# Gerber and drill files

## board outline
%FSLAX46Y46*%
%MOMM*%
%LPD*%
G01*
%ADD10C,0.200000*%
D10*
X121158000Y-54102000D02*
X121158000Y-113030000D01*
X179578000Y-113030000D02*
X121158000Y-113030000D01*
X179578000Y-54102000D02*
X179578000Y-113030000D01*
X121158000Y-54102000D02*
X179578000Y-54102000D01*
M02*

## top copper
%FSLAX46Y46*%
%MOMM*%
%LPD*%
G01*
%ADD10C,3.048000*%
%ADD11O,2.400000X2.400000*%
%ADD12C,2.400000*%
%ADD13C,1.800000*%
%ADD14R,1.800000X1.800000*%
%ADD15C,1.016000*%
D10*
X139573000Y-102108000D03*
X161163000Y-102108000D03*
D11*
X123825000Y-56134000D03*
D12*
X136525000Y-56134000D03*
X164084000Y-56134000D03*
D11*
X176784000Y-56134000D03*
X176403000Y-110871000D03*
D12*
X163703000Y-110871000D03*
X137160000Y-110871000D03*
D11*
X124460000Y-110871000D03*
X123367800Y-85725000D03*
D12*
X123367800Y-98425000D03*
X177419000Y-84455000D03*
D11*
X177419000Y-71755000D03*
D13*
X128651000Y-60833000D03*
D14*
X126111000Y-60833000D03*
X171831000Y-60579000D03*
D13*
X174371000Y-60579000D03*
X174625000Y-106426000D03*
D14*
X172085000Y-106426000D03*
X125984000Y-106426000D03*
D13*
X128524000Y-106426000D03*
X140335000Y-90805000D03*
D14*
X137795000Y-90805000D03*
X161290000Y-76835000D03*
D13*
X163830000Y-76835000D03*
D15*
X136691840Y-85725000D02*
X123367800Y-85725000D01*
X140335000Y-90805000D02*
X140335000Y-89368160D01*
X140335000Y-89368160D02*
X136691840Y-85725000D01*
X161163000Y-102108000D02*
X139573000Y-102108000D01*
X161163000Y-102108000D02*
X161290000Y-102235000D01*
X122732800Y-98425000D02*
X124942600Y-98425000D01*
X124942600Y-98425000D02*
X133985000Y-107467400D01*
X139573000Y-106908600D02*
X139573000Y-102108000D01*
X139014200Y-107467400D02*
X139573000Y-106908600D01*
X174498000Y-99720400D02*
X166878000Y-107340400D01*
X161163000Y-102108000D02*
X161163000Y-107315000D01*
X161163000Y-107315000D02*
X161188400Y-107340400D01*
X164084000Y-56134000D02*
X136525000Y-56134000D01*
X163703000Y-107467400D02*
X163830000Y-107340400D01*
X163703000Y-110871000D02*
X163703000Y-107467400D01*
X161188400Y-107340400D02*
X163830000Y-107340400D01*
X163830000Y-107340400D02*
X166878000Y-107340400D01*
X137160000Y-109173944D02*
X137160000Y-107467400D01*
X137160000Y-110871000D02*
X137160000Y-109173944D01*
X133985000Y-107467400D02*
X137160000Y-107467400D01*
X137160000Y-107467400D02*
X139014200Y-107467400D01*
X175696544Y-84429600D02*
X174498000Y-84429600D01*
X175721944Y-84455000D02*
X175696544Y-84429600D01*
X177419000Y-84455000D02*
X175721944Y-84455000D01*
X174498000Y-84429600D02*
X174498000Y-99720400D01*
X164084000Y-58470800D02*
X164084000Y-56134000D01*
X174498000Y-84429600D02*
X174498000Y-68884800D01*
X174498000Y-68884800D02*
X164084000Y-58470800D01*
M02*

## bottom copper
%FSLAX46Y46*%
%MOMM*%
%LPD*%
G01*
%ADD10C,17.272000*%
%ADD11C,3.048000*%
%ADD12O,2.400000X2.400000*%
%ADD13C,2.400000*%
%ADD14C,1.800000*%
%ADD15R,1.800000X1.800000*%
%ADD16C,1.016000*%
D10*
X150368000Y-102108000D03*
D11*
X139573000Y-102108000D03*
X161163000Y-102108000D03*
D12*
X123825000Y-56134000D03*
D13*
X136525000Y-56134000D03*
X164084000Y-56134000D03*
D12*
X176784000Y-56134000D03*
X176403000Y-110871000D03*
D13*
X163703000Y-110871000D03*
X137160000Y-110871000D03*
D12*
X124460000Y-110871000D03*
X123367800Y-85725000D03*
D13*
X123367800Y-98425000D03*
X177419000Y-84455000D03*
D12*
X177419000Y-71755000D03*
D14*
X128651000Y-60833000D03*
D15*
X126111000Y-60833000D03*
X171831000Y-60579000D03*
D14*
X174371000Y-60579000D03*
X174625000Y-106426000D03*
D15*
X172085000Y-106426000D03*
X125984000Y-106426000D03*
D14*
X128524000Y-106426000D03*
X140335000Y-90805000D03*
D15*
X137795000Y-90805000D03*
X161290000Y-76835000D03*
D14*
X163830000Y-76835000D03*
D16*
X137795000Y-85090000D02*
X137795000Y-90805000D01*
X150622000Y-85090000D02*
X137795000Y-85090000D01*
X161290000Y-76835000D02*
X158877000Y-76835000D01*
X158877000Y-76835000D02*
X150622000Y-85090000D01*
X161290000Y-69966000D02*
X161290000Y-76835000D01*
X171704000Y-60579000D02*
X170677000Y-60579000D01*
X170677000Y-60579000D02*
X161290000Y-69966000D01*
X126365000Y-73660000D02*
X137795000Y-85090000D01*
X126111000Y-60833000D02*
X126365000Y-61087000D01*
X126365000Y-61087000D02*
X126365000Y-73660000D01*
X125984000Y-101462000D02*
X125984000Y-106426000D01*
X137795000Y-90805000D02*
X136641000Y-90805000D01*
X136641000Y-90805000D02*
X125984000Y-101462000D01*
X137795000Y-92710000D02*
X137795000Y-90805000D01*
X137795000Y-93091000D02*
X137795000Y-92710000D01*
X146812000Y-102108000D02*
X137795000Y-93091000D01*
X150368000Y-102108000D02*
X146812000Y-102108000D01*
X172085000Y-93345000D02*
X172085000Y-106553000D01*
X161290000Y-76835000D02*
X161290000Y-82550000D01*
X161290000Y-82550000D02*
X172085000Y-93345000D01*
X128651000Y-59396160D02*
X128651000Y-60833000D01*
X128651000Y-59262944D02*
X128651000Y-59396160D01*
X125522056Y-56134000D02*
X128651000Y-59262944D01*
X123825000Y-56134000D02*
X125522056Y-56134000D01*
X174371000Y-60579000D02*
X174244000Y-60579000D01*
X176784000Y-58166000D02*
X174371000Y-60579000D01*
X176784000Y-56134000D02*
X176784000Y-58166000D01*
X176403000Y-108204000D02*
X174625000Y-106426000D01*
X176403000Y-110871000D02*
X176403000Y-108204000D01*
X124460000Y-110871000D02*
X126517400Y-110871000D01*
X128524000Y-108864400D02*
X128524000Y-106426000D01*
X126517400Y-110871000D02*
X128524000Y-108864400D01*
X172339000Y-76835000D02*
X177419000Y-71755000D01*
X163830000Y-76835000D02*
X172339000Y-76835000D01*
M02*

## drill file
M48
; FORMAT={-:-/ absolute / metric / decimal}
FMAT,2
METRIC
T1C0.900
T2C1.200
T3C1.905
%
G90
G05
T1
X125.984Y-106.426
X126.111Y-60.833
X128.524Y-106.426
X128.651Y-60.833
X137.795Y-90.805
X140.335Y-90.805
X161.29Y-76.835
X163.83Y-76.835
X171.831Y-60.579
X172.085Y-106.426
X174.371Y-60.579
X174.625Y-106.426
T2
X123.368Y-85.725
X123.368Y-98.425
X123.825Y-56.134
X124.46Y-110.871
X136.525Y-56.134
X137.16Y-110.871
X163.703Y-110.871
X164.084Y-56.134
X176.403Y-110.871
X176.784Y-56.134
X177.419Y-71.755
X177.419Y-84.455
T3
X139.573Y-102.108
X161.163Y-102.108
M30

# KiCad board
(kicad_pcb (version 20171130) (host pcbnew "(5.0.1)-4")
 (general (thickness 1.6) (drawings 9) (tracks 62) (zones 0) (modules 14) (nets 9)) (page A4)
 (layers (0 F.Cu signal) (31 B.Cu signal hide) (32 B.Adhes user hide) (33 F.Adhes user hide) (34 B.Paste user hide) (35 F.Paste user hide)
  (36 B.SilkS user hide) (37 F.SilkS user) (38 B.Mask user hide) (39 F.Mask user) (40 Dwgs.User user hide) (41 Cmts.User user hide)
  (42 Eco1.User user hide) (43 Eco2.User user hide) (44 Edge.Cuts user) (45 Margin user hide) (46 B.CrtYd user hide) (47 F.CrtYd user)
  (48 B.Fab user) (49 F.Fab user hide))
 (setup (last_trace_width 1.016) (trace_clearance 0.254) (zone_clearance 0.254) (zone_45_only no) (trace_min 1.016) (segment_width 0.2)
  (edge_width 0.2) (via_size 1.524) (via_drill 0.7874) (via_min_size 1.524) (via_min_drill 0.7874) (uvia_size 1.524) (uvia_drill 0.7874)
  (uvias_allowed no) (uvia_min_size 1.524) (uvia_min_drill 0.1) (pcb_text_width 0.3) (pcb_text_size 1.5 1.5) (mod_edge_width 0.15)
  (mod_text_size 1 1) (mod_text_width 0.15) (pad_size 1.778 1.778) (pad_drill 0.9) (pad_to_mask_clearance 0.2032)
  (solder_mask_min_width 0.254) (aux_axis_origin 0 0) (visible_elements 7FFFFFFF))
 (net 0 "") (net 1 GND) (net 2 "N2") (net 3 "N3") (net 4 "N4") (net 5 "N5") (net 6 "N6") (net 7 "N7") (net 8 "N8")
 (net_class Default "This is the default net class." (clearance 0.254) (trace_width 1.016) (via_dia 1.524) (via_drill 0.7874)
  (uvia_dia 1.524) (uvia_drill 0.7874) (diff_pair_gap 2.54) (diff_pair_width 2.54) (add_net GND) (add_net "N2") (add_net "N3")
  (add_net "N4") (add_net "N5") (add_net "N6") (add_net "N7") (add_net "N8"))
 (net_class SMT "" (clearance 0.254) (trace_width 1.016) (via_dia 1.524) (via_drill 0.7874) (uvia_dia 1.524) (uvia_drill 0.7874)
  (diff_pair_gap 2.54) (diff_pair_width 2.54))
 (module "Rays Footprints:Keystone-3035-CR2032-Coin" (layer B.Cu) (at 150.368 102.108 180)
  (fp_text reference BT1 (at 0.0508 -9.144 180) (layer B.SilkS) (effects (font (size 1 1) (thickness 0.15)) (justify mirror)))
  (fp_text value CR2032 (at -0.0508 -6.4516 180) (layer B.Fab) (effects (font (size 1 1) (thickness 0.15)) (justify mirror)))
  (pad 2 smd circle (at 0 0 180) (size 17.272 17.272) (layers B.Cu B.Paste B.Mask) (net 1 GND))
  (pad 1 thru_hole circle (at 10.795 0 180) (size 3.048 3.048) (drill 1.905) (layers *.Cu *.Mask) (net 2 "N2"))
  (pad 1 thru_hole circle (at -10.795 0 90) (size 3.048 3.048) (drill 1.905) (layers *.Cu *.Mask) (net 2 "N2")))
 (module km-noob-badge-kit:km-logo (layer F.Cu) (at 150.368 83.566)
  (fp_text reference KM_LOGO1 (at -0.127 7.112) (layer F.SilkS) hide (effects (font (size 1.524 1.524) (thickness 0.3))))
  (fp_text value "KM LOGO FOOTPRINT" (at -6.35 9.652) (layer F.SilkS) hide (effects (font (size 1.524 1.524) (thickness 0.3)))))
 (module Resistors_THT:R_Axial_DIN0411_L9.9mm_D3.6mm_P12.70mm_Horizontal (layer F.Cu) (at 136.525 56.134 180)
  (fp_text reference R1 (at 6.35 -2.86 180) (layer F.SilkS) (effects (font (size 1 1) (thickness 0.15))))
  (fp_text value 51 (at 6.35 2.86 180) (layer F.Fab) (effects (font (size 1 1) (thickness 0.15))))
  (pad 2 thru_hole oval (at 12.7 0 180) (size 2.4 2.4) (drill 1.2) (layers *.Cu *.Mask) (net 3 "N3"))
  (pad 1 thru_hole circle (at 0 0 180) (size 2.4 2.4) (drill 1.2) (layers *.Cu *.Mask) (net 2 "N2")))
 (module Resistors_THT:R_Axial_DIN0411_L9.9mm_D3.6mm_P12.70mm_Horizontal (layer F.Cu) (at 164.084 56.134)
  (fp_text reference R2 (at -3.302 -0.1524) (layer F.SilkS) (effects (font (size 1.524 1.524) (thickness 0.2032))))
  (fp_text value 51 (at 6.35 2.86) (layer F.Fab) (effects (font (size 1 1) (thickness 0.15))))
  (pad 1 thru_hole circle (at 0 0) (size 2.4 2.4) (drill 1.2) (layers *.Cu *.Mask) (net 2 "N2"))
  (pad 2 thru_hole oval (at 12.7 0) (size 2.4 2.4) (drill 1.2) (layers *.Cu *.Mask) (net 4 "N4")))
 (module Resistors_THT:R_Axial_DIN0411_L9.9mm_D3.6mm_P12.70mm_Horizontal (layer F.Cu) (at 163.703 110.871)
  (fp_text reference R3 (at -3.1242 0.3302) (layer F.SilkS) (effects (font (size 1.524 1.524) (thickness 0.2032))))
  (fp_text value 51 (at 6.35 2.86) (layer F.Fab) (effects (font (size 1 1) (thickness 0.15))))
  (pad 2 thru_hole oval (at 12.7 0) (size 2.4 2.4) (drill 1.2) (layers *.Cu *.Mask) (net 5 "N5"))
  (pad 1 thru_hole circle (at 0 0) (size 2.4 2.4) (drill 1.2) (layers *.Cu *.Mask) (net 2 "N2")))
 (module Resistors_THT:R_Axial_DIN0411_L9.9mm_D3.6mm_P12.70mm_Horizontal (layer F.Cu) (at 137.16 110.871 180)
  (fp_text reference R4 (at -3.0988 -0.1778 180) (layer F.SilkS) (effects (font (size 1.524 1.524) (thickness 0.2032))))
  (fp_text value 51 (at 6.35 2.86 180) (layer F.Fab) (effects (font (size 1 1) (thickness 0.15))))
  (pad 1 thru_hole circle (at 0 0 180) (size 2.4 2.4) (drill 1.2) (layers *.Cu *.Mask) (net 2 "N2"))
  (pad 2 thru_hole oval (at 12.7 0 180) (size 2.4 2.4) (drill 1.2) (layers *.Cu *.Mask) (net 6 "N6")))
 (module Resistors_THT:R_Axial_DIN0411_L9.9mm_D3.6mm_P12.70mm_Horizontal (layer F.Cu) (at 123.3678 98.425 90)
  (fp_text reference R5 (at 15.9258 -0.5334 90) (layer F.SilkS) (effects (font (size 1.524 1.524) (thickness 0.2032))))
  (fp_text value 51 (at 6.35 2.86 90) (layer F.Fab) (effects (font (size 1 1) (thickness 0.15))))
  (pad 2 thru_hole oval (at 12.7 0 90) (size 2.4 2.4) (drill 1.2) (layers *.Cu *.Mask) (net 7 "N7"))
  (pad 1 thru_hole circle (at 0 0 90) (size 2.4 2.4) (drill 1.2) (layers *.Cu *.Mask) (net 2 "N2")))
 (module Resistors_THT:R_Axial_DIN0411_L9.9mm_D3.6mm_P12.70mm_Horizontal (layer F.Cu) (at 177.419 84.455 90)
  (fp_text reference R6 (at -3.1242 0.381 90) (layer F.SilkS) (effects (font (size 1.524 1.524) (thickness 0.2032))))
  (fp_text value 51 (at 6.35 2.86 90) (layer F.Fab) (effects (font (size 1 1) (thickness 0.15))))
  (pad 1 thru_hole circle (at 0 0 90) (size 2.4 2.4) (drill 1.2) (layers *.Cu *.Mask) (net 2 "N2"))
  (pad 2 thru_hole oval (at 12.7 0 90) (size 2.4 2.4) (drill 1.2) (layers *.Cu *.Mask) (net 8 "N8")))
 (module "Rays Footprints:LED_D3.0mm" (layer F.Cu) (at 126.111 60.833)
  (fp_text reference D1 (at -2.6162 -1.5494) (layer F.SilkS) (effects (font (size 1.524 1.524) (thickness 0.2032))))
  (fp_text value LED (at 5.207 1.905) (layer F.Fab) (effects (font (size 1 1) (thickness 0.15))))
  (pad 2 thru_hole circle (at 2.54 0) (size 1.8 1.8) (drill 0.9) (layers *.Cu *.Mask) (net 3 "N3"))
  (pad 1 thru_hole rect (at 0 0) (size 1.8 1.8) (drill 0.9) (layers *.Cu *.Mask) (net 1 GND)))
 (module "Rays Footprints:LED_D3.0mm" (layer F.Cu) (at 171.831 60.579)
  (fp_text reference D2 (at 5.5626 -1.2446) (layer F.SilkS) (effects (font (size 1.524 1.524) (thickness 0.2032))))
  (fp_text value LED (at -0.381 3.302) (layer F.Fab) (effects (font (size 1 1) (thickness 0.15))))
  (pad 1 thru_hole rect (at 0 0) (size 1.8 1.8) (drill 0.9) (layers *.Cu *.Mask) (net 1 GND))
  (pad 2 thru_hole circle (at 2.54 0) (size 1.8 1.8) (drill 0.9) (layers *.Cu *.Mask) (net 4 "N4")))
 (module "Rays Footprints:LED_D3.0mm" (layer F.Cu) (at 172.085 106.426)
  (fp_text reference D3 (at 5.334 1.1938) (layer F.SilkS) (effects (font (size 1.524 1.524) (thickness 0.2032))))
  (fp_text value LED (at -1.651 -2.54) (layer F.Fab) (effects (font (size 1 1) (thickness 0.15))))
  (pad 2 thru_hole circle (at 2.54 0) (size 1.8 1.8) (drill 0.9) (layers *.Cu *.Mask) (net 5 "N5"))
  (pad 1 thru_hole rect (at 0 0) (size 1.8 1.8) (drill 0.9) (layers *.Cu *.Mask) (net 1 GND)))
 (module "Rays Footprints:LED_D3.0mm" (layer F.Cu) (at 125.984 106.426)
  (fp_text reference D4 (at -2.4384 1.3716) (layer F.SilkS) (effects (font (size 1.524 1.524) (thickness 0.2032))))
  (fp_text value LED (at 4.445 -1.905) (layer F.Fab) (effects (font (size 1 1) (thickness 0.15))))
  (pad 1 thru_hole rect (at 0 0) (size 1.8 1.8) (drill 0.9) (layers *.Cu *.Mask) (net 1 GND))
  (pad 2 thru_hole circle (at 2.54 0) (size 1.8 1.8) (drill 0.9) (layers *.Cu *.Mask) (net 6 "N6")))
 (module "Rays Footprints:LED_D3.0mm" (layer F.Cu) (at 137.795 90.805)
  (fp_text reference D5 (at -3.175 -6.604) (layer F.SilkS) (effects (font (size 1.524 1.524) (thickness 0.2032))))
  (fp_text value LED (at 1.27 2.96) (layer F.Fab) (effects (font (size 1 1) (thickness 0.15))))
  (pad 2 thru_hole circle (at 2.54 0) (size 1.8 1.8) (drill 0.9) (layers *.Cu *.Mask) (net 7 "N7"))
  (pad 1 thru_hole rect (at 0 0) (size 1.8 1.8) (drill 0.9) (layers *.Cu *.Mask) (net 1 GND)))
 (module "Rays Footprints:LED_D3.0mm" (layer F.Cu) (at 161.29 76.835)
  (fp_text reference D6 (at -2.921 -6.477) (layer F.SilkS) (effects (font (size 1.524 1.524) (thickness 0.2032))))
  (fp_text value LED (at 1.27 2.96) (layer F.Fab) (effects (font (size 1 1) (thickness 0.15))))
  (pad 1 thru_hole rect (at 0 0) (size 1.8 1.8) (drill 0.9) (layers *.Cu *.Mask) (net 1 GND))
  (pad 2 thru_hole circle (at 2.54 0) (size 1.8 1.8) (drill 0.9) (layers *.Cu *.Mask) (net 8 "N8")))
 (gr_line (start 121.158 54.102) (end 121.158 113.03) (layer Edge.Cuts) (width 0.2))
 (gr_line (start 179.578 113.03) (end 121.158 113.03) (layer Edge.Cuts) (width 0.2))
 (gr_line (start 179.578 54.102) (end 179.578 113.03) (layer Edge.Cuts) (width 0.2))
 (gr_line (start 121.158 54.102) (end 179.578 54.102) (layer Edge.Cuts) (width 0.2))
 (segment (start 137.795 85.09) (end 137.795 90.805) (width 1.016) (layer B.Cu) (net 1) (status 20))
 (segment (start 150.622 85.09) (end 137.795 85.09) (width 1.016) (layer B.Cu) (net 1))
 (segment (start 161.29 76.835) (end 158.877 76.835) (width 1.016) (layer B.Cu) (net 1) (status 10))
 (segment (start 158.877 76.835) (end 150.622 85.09) (width 1.016) (layer B.Cu) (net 1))
 (segment (start 161.29 69.966) (end 161.29 76.835) (width 1.016) (layer B.Cu) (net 1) (status 20))
 (segment (start 171.704 60.579) (end 170.677 60.579) (width 1.016) (layer B.Cu) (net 1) (status 10))
 (segment (start 170.677 60.579) (end 161.29 69.966) (width 1.016) (layer B.Cu) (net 1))
 (segment (start 126.365 73.66) (end 137.795 85.09) (width 1.016) (layer B.Cu) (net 1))
 (segment (start 126.111 60.833) (end 126.365 61.087) (width 1.016) (layer B.Cu) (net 1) (status 30))
 (segment (start 126.365 61.087) (end 126.365 73.66) (width 1.016) (layer B.Cu) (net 1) (status 10))
 (segment (start 125.984 101.462) (end 125.984 106.426) (width 1.016) (layer B.Cu) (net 1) (status 20))
 (segment (start 137.795 90.805) (end 136.641 90.805) (width 1.016) (layer B.Cu) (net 1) (status 10))
 (segment (start 136.641 90.805) (end 125.984 101.462) (width 1.016) (layer B.Cu) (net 1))
 (segment (start 137.795 92.71) (end 137.795 90.805) (width 1.016) (layer B.Cu) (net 1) (status 20))
 (segment (start 137.795 93.091) (end 137.795 92.71) (width 1.016) (layer B.Cu) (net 1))
 (segment (start 146.812 102.108) (end 137.795 93.091) (width 1.016) (layer B.Cu) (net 1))
 (segment (start 150.368 102.108) (end 146.812 102.108) (width 1.016) (layer B.Cu) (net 1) (status 10))
 (segment (start 172.085 93.345) (end 172.085 106.553) (width 1.016) (layer B.Cu) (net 1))
 (segment (start 161.29 76.835) (end 161.29 82.55) (width 1.016) (layer B.Cu) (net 1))
 (segment (start 161.29 82.55) (end 172.085 93.345) (width 1.016) (layer B.Cu) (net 1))
 (segment (start 128.651 59.39616) (end 128.651 60.833) (width 1.016) (layer B.Cu) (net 3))
 (segment (start 128.651 59.262944) (end 128.651 59.39616) (width 1.016) (layer B.Cu) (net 3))
 (segment (start 125.522056 56.134) (end 128.651 59.262944) (width 1.016) (layer B.Cu) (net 3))
 (segment (start 123.825 56.134) (end 125.522056 56.134) (width 1.016) (layer B.Cu) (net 3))
 (segment (start 174.371 60.579) (end 174.244 60.579) (width 1.016) (layer B.Cu) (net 4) (status 30))
 (segment (start 176.784 58.166) (end 174.371 60.579) (width 1.016) (layer B.Cu) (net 4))
 (segment (start 176.784 56.134) (end 176.784 58.166) (width 1.016) (layer B.Cu) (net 4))
 (segment (start 176.403 108.204) (end 174.625 106.426) (width 1.016) (layer B.Cu) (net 5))
 (segment (start 176.403 110.871) (end 176.403 108.204) (width 1.016) (layer B.Cu) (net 5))
 (segment (start 124.46 110.871) (end 126.5174 110.871) (width 1.016) (layer B.Cu) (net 6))
 (segment (start 128.524 108.8644) (end 128.524 106.426) (width 1.016) (layer B.Cu) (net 6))
 (segment (start 126.5174 110.871) (end 128.524 108.8644) (width 1.016) (layer B.Cu) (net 6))
 (segment (start 136.69184 85.725) (end 123.3678 85.725) (width 1.016) (layer F.Cu) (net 7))
 (segment (start 140.335 90.805) (end 140.335 89.36816) (width 1.016) (layer F.Cu) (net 7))
 (segment (start 140.335 89.36816) (end 136.69184 85.725) (width 1.016) (layer F.Cu) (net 7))
 (segment (start 172.339 76.835) (end 177.419 71.755) (width 1.016) (layer B.Cu) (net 8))
 (segment (start 163.83 76.835) (end 172.339 76.835) (width 1.016) (layer B.Cu) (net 8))
 (segment (start 161.163 102.108) (end 139.573 102.108) (width 1.016) (layer F.Cu) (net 2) (status 30))
 (segment (start 161.163 102.108) (end 161.29 102.235) (width 1.016) (layer F.Cu) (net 2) (status 30))
 (segment (start 122.7328 98.425) (end 124.9426 98.425) (width 1.016) (layer F.Cu) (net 2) (status 10))
 (segment (start 124.9426 98.425) (end 133.985 107.4674) (width 1.016) (layer F.Cu) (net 2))
 (segment (start 139.573 106.9086) (end 139.573 102.108) (width 1.016) (layer F.Cu) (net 2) (status 20))
 (segment (start 139.0142 107.4674) (end 139.573 106.9086) (width 1.016) (layer F.Cu) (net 2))
 (segment (start 174.498 99.7204) (end 166.878 107.3404) (width 1.016) (layer F.Cu) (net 2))
 (segment (start 161.163 102.108) (end 161.163 107.315) (width 1.016) (layer F.Cu) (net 2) (status 10))
 (segment (start 161.163 107.315) (end 161.1884 107.3404) (width 1.016) (layer F.Cu) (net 2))
 (segment (start 164.084 56.134) (end 136.525 56.134) (width 1.016) (layer F.Cu) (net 2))
 (segment (start 163.703 107.4674) (end 163.83 107.3404) (width 1.016) (layer F.Cu) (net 2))
 (segment (start 163.703 110.871) (end 163.703 107.4674) (width 1.016) (layer F.Cu) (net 2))
 (segment (start 161.1884 107.3404) (end 163.83 107.3404) (width 1.016) (layer F.Cu) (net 2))
 (segment (start 163.83 107.3404) (end 166.878 107.3404) (width 1.016) (layer F.Cu) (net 2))
 (segment (start 137.16 109.173944) (end 137.16 107.4674) (width 1.016) (layer F.Cu) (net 2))
 (segment (start 137.16 110.871) (end 137.16 109.173944) (width 1.016) (layer F.Cu) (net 2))
 (segment (start 133.985 107.4674) (end 137.16 107.4674) (width 1.016) (layer F.Cu) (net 2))
 (segment (start 137.16 107.4674) (end 139.0142 107.4674) (width 1.016) (layer F.Cu) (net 2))
 (segment (start 175.696544 84.4296) (end 174.498 84.4296) (width 1.016) (layer F.Cu) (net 2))
 (segment (start 175.721944 84.455) (end 175.696544 84.4296) (width 1.016) (layer F.Cu) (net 2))
 (segment (start 177.419 84.455) (end 175.721944 84.455) (width 1.016) (layer F.Cu) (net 2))
 (segment (start 174.498 84.4296) (end 174.498 99.7204) (width 1.016) (layer F.Cu) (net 2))
 (segment (start 164.084 58.4708) (end 164.084 56.134) (width 1.016) (layer F.Cu) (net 2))
 (segment (start 174.498 84.4296) (end 174.498 68.8848) (width 1.016) (layer F.Cu) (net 2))
 (segment (start 174.498 68.8848) (end 164.084 58.4708) (width 1.016) (layer F.Cu) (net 2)))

